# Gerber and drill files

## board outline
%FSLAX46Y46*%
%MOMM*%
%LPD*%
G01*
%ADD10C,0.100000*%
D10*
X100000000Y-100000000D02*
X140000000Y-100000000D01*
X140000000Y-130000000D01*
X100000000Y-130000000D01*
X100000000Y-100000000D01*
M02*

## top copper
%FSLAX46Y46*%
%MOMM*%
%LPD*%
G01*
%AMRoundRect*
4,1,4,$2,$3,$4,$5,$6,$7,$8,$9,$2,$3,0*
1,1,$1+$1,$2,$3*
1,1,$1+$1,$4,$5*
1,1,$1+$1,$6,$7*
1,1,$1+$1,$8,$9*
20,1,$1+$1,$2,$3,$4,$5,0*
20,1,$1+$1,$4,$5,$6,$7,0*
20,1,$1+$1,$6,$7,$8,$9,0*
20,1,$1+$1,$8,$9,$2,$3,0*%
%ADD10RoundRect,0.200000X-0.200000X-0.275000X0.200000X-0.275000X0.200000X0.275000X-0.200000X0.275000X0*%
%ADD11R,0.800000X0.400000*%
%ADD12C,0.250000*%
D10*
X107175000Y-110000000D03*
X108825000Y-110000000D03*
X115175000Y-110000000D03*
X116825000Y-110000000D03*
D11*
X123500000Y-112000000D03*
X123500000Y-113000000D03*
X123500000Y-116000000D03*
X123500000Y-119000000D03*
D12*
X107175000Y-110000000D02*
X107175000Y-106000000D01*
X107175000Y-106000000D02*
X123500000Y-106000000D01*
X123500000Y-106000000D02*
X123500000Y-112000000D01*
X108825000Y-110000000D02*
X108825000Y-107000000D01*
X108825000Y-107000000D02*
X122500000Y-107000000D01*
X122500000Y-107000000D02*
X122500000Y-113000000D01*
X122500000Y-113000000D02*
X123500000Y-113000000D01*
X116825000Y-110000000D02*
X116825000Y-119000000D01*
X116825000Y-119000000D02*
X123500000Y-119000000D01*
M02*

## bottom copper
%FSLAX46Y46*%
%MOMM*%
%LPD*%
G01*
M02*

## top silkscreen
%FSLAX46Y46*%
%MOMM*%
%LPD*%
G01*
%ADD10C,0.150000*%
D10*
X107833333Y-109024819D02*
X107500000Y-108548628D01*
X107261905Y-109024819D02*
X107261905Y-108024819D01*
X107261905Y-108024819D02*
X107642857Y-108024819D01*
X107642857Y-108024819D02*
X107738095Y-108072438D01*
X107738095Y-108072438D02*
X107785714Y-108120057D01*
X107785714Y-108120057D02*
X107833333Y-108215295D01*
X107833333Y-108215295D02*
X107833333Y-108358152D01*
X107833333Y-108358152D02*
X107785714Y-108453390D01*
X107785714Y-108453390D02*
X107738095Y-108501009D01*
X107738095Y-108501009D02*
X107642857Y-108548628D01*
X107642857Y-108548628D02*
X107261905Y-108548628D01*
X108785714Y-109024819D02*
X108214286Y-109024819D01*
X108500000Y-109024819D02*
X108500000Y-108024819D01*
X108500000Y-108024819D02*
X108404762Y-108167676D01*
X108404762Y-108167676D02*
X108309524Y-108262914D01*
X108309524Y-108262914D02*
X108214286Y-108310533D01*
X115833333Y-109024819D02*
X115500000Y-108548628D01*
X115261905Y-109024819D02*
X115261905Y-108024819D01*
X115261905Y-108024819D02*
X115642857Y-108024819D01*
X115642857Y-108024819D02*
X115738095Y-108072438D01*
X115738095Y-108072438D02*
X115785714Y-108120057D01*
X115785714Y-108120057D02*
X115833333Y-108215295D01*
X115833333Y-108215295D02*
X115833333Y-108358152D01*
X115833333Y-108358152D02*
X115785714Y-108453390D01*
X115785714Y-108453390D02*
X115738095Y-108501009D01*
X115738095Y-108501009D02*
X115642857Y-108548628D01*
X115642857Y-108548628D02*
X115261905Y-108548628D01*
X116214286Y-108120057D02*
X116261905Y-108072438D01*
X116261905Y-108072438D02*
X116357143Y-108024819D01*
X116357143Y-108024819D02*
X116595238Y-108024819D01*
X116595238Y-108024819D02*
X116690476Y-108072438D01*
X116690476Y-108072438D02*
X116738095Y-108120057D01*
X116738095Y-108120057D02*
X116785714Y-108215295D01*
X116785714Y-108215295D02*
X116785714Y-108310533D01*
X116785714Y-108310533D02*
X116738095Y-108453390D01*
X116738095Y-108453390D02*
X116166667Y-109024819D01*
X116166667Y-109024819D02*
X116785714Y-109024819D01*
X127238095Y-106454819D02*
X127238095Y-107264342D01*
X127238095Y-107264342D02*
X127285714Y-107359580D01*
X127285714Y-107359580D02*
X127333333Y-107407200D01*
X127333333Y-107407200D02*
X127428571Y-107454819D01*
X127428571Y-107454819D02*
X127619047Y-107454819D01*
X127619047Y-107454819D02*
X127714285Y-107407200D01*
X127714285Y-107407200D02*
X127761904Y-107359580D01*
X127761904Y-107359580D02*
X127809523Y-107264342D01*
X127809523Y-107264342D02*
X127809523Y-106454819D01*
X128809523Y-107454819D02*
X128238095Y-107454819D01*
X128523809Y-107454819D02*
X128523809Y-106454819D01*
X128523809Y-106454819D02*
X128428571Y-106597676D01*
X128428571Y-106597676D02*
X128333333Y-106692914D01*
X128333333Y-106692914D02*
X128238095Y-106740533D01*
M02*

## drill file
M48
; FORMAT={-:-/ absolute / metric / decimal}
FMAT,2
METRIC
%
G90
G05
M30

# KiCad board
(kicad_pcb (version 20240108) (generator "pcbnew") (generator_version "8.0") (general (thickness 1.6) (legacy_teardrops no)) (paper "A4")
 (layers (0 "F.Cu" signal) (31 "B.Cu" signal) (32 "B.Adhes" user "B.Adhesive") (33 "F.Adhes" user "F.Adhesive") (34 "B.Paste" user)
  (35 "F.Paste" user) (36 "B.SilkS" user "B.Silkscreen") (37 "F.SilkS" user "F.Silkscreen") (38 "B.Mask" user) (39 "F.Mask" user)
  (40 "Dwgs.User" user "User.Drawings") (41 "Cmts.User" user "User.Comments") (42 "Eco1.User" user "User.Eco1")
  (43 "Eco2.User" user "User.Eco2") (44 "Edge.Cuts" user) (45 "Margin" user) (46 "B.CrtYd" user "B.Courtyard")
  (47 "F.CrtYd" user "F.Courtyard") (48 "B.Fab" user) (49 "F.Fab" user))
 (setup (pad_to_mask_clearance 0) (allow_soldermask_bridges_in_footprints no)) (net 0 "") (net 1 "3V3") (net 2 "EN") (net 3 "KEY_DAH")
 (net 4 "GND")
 (gr_rect (start 100 100) (end 140 130) (stroke (width 0.1) (type default)) (layer "Edge.Cuts"))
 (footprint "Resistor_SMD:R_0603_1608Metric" (layer "F.Cu") (at 108 110)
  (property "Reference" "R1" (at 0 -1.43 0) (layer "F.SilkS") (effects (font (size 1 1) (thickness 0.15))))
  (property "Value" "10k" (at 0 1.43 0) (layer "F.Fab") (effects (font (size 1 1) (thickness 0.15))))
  (pad "1" smd roundrect (at -0.825 0) (size 0.8 0.95) (layers "F.Cu" "F.Paste" "F.Mask") (roundrect_rratio 0.25) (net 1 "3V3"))
  (pad "2" smd roundrect (at 0.825 0) (size 0.8 0.95) (layers "F.Cu" "F.Paste" "F.Mask") (roundrect_rratio 0.25) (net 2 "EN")))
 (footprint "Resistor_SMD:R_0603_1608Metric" (layer "F.Cu") (at 116 110)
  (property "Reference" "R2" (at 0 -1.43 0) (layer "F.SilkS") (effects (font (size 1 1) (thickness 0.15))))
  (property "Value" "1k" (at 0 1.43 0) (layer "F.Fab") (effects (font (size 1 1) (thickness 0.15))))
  (pad "1" smd roundrect (at -0.825 0) (size 0.8 0.95) (layers "F.Cu" "F.Paste" "F.Mask") (roundrect_rratio 0.25) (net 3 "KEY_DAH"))
  (pad "2" smd roundrect (at 0.825 0) (size 0.8 0.95) (layers "F.Cu" "F.Paste" "F.Mask") (roundrect_rratio 0.25) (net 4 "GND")))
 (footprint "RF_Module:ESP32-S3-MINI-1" (layer "F.Cu") (at 128 115)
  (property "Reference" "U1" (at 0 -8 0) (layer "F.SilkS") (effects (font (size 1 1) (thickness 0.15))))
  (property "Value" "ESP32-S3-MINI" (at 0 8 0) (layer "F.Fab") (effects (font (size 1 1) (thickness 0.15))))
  (pad "1" smd rect (at -4.5 -3.0) (size 0.8 0.4) (layers "F.Cu" "F.Paste" "F.Mask") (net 1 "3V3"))
  (pad "2" smd rect (at -4.5 -2.0) (size 0.8 0.4) (layers "F.Cu" "F.Paste" "F.Mask") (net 2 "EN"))
  (pad "5" smd rect (at -4.5 1.0) (size 0.8 0.4) (layers "F.Cu" "F.Paste" "F.Mask") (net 3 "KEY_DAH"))
  (pad "8" smd rect (at -4.5 4.0) (size 0.8 0.4) (layers "F.Cu" "F.Paste" "F.Mask") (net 4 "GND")))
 (segment (start 107.175 110) (end 107.175 106) (width 0.25) (layer "F.Cu") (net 1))
 (segment (start 107.175 106) (end 123.5 106) (width 0.25) (layer "F.Cu") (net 1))
 (segment (start 123.5 106) (end 123.5 112) (width 0.25) (layer "F.Cu") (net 1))
 (segment (start 108.825 110) (end 108.825 107) (width 0.25) (layer "F.Cu") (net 2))
 (segment (start 108.825 107) (end 122.5 107) (width 0.25) (layer "F.Cu") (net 2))
 (segment (start 122.5 107) (end 122.5 113) (width 0.25) (layer "F.Cu") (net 2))
 (segment (start 122.5 113) (end 123.5 113) (width 0.25) (layer "F.Cu") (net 2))
 (segment (start 116.825 110) (end 116.825 119) (width 0.25) (layer "F.Cu") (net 4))
 (segment (start 116.825 119) (end 123.5 119) (width 0.25) (layer "F.Cu") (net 4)))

